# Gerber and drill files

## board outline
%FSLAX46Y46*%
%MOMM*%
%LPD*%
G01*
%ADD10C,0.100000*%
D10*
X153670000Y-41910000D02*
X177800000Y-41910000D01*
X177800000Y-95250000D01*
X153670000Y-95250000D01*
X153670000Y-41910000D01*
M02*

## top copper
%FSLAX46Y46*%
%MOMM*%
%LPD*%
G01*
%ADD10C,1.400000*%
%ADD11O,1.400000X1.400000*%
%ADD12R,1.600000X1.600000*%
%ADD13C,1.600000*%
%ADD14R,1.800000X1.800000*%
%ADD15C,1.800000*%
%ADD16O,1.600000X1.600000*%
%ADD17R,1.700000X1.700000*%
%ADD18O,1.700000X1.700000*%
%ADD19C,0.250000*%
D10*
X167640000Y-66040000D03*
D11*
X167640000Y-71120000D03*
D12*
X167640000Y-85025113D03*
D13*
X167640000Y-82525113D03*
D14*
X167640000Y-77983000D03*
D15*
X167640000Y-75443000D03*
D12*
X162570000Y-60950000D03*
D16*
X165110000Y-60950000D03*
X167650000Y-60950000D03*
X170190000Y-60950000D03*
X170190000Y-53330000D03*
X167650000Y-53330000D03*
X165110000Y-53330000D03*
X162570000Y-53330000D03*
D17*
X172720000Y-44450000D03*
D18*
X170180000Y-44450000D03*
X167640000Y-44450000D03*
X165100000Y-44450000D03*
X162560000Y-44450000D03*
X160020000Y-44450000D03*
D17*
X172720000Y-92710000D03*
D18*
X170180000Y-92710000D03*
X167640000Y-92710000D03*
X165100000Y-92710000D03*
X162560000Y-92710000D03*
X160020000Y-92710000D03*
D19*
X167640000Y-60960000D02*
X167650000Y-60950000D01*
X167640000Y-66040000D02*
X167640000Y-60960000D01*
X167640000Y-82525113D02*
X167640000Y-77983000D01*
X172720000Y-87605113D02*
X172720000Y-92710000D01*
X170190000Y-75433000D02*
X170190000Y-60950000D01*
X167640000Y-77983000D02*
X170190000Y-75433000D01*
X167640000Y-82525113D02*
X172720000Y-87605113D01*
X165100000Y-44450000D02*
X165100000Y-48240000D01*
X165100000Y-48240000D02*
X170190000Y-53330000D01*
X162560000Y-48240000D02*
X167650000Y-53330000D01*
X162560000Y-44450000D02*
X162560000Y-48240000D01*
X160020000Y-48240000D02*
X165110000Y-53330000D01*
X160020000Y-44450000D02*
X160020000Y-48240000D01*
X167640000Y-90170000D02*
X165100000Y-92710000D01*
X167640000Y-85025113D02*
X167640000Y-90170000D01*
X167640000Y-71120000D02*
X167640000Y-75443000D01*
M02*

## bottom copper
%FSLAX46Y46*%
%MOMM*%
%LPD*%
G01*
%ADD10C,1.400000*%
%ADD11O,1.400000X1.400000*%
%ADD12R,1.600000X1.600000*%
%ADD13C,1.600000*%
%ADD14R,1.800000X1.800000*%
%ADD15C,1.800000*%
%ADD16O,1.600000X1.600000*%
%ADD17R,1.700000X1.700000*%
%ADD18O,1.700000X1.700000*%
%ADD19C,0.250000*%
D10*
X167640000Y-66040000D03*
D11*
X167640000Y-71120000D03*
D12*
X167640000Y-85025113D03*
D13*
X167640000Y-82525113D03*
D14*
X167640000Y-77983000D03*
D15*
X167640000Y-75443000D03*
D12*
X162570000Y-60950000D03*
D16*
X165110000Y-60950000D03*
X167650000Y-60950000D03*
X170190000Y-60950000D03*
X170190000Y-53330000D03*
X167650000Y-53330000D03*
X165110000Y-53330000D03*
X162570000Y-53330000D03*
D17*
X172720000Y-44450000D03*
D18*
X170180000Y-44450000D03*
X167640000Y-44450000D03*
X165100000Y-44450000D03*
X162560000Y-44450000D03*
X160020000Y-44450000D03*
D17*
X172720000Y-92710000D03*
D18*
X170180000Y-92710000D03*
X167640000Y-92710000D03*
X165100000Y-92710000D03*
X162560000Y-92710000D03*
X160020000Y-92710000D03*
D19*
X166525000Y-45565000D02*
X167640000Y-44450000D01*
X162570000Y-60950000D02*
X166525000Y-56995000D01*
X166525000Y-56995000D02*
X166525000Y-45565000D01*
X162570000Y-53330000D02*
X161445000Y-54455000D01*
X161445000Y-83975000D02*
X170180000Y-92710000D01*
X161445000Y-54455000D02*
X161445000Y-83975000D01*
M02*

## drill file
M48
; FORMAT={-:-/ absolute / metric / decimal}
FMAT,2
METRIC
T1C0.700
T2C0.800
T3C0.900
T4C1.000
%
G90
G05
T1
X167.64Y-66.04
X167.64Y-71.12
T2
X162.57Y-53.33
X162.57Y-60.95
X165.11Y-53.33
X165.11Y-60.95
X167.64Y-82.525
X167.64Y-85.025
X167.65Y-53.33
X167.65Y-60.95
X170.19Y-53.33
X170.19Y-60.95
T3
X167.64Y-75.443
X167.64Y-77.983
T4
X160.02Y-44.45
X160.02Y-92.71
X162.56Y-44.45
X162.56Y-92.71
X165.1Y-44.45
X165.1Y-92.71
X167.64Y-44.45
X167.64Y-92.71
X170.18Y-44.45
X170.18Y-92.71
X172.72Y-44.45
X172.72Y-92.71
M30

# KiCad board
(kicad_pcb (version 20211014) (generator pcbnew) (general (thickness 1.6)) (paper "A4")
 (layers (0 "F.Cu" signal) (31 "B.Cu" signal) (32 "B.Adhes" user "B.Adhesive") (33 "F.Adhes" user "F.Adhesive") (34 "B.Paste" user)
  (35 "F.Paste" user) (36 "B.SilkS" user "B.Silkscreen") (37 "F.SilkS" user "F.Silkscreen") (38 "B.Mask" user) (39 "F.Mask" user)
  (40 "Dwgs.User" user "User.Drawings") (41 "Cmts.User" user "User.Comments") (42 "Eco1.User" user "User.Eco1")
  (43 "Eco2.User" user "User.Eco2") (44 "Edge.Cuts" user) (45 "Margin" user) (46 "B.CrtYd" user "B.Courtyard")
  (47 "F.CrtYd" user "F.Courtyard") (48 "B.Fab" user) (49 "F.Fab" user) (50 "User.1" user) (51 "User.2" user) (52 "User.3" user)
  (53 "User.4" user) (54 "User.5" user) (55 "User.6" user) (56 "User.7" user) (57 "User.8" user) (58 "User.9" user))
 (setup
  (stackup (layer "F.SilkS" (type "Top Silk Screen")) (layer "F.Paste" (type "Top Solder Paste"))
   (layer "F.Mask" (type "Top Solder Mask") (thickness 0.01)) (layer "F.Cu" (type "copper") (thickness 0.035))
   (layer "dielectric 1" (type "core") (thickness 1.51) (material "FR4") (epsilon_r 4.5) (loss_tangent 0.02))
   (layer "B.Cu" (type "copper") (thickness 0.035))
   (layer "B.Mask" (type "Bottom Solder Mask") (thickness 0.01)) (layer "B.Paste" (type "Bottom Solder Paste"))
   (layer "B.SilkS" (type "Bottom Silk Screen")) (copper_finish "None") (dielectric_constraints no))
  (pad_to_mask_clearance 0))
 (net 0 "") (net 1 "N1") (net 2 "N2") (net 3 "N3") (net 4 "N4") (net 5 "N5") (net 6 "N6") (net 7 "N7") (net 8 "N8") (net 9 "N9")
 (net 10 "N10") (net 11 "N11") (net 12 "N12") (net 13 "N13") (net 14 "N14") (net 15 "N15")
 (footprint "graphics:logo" (layer "F.Cu") (at 158.75 86.36 90)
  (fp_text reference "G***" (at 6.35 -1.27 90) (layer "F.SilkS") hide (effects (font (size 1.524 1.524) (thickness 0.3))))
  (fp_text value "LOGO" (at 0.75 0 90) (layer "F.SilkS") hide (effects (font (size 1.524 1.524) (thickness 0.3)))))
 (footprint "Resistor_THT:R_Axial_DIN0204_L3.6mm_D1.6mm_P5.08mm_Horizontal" (layer "F.Cu") (at 167.64 66.04 -90)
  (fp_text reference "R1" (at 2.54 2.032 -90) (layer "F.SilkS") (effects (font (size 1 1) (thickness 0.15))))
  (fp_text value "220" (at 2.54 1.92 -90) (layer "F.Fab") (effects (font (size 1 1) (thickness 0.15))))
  (pad "1" thru_hole circle (at 0 0 270) (size 1.4 1.4) (drill 0.7) (layers *.Cu *.Mask) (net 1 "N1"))
  (pad "2" thru_hole oval (at 5.08 0 270) (size 1.4 1.4) (drill 0.7) (layers *.Cu *.Mask) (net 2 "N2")))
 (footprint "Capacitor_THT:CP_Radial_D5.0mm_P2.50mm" (layer "F.Cu") (at 167.64 85.025113 90)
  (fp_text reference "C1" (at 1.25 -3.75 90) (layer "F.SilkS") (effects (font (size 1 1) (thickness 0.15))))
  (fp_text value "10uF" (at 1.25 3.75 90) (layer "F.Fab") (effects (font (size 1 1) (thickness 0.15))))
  (pad "1" thru_hole rect (at 0 0 90) (size 1.6 1.6) (drill 0.8) (layers *.Cu *.Mask) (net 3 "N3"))
  (pad "2" thru_hole circle (at 2.5 0 90) (size 1.6 1.6) (drill 0.8) (layers *.Cu *.Mask) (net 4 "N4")))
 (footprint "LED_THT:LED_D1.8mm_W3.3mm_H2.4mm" (layer "F.Cu") (at 167.64 77.983 90)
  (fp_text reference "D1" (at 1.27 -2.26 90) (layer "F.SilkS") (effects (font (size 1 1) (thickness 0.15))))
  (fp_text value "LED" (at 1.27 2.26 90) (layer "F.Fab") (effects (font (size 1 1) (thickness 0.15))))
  (pad "1" thru_hole rect (at 0 0 90) (size 1.8 1.8) (drill 0.9) (layers *.Cu *.Mask) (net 4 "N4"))
  (pad "2" thru_hole circle (at 2.54 0 90) (size 1.8 1.8) (drill 0.9) (layers *.Cu *.Mask) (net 2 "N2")))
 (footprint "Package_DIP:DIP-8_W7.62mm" (layer "F.Cu") (at 162.57 60.95 90)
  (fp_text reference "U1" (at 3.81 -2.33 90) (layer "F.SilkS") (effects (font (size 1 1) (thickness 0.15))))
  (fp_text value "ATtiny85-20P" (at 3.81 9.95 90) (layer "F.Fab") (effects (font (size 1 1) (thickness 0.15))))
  (pad "1" thru_hole rect (at 0 0 90) (size 1.6 1.6) (drill 0.8) (layers *.Cu *.Mask) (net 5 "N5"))
  (pad "2" thru_hole oval (at 0 2.54 90) (size 1.6 1.6) (drill 0.8) (layers *.Cu *.Mask) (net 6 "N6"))
  (pad "3" thru_hole oval (at 0 5.08 90) (size 1.6 1.6) (drill 0.8) (layers *.Cu *.Mask) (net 1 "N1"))
  (pad "4" thru_hole oval (at 0 7.62 90) (size 1.6 1.6) (drill 0.8) (layers *.Cu *.Mask) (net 4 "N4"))
  (pad "5" thru_hole oval (at 7.62 7.62 90) (size 1.6 1.6) (drill 0.8) (layers *.Cu *.Mask) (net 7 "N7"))
  (pad "6" thru_hole oval (at 7.62 5.08 90) (size 1.6 1.6) (drill 0.8) (layers *.Cu *.Mask) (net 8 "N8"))
  (pad "7" thru_hole oval (at 7.62 2.54 90) (size 1.6 1.6) (drill 0.8) (layers *.Cu *.Mask) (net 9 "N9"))
  (pad "8" thru_hole oval (at 7.62 0 90) (size 1.6 1.6) (drill 0.8) (layers *.Cu *.Mask) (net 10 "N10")))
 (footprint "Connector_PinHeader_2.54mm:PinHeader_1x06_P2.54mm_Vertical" (layer "B.Cu") (at 172.72 44.45 90)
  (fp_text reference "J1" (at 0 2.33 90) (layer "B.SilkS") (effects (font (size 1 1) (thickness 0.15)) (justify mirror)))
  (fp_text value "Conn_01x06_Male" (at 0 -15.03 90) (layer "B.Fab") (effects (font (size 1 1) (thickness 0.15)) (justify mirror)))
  (pad "1" thru_hole rect (at 0 0 90) (size 1.7 1.7) (drill 1) (layers *.Cu *.Mask) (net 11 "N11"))
  (pad "2" thru_hole oval (at 0 -2.54 90) (size 1.7 1.7) (drill 1) (layers *.Cu *.Mask) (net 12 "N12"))
  (pad "3" thru_hole oval (at 0 -5.08 90) (size 1.7 1.7) (drill 1) (layers *.Cu *.Mask) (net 5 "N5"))
  (pad "4" thru_hole oval (at 0 -7.62 90) (size 1.7 1.7) (drill 1) (layers *.Cu *.Mask) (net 7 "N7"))
  (pad "5" thru_hole oval (at 0 -10.16 90) (size 1.7 1.7) (drill 1) (layers *.Cu *.Mask) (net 8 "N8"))
  (pad "6" thru_hole oval (at 0 -12.7 90) (size 1.7 1.7) (drill 1) (layers *.Cu *.Mask) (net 9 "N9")))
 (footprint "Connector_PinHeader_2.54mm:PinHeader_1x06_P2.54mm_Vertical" (layer "B.Cu") (at 172.72 92.71 90)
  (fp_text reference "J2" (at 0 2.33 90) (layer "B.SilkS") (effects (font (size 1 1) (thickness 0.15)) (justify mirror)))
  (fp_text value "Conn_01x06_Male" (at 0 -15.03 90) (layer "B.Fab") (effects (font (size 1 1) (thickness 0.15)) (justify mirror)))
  (pad "1" thru_hole rect (at 0 0 90) (size 1.7 1.7) (drill 1) (layers *.Cu *.Mask) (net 4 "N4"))
  (pad "2" thru_hole oval (at 0 -2.54 90) (size 1.7 1.7) (drill 1) (layers *.Cu *.Mask) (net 10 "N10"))
  (pad "3" thru_hole oval (at 0 -5.08 90) (size 1.7 1.7) (drill 1) (layers *.Cu *.Mask) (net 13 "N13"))
  (pad "4" thru_hole oval (at 0 -7.62 90) (size 1.7 1.7) (drill 1) (layers *.Cu *.Mask) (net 3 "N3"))
  (pad "5" thru_hole oval (at 0 -10.16 90) (size 1.7 1.7) (drill 1) (layers *.Cu *.Mask) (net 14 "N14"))
  (pad "6" thru_hole oval (at 0 -12.7 90) (size 1.7 1.7) (drill 1) (layers *.Cu *.Mask) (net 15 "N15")))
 (gr_rect (start 153.67 41.91) (end 177.8 95.25) (layer "Edge.Cuts") (width 0.1) (fill none))
 (segment (start 166.525 45.565) (end 167.64 44.45) (width 0.25) (layer "B.Cu") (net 5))
 (segment (start 162.57 60.95) (end 166.525 56.995) (width 0.25) (layer "B.Cu") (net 5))
 (segment (start 166.525 56.995) (end 166.525 45.565) (width 0.25) (layer "B.Cu") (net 5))
 (segment (start 167.64 60.96) (end 167.65 60.95) (width 0.25) (layer "F.Cu") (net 1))
 (segment (start 167.64 66.04) (end 167.64 60.96) (width 0.25) (layer "F.Cu") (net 1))
 (segment (start 167.64 82.525113) (end 167.64 77.983) (width 0.25) (layer "F.Cu") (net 4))
 (segment (start 172.72 87.605113) (end 172.72 92.71) (width 0.25) (layer "F.Cu") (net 4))
 (segment (start 170.19 75.433) (end 170.19 60.95) (width 0.25) (layer "F.Cu") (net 4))
 (segment (start 167.64 77.983) (end 170.19 75.433) (width 0.25) (layer "F.Cu") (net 4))
 (segment (start 167.64 82.525113) (end 172.72 87.605113) (width 0.25) (layer "F.Cu") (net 4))
 (segment (start 165.1 44.45) (end 165.1 48.24) (width 0.25) (layer "F.Cu") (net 7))
 (segment (start 165.1 48.24) (end 170.19 53.33) (width 0.25) (layer "F.Cu") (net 7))
 (segment (start 162.56 48.24) (end 167.65 53.33) (width 0.25) (layer "F.Cu") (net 8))
 (segment (start 162.56 44.45) (end 162.56 48.24) (width 0.25) (layer "F.Cu") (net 8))
 (segment (start 160.02 48.24) (end 165.11 53.33) (width 0.25) (layer "F.Cu") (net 9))
 (segment (start 160.02 44.45) (end 160.02 48.24) (width 0.25) (layer "F.Cu") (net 9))
 (segment (start 162.57 53.33) (end 161.445 54.455) (width 0.25) (layer "B.Cu") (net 10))
 (segment (start 161.445 83.975) (end 170.18 92.71) (width 0.25) (layer "B.Cu") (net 10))
 (segment (start 161.445 54.455) (end 161.445 83.975) (width 0.25) (layer "B.Cu") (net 10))
 (segment (start 167.64 90.17) (end 165.1 92.71) (width 0.25) (layer "F.Cu") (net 3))
 (segment (start 167.64 85.025113) (end 167.64 90.17) (width 0.25) (layer "F.Cu") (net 3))
 (segment (start 167.64 71.12) (end 167.64 75.443) (width 0.25) (layer "F.Cu") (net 2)))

